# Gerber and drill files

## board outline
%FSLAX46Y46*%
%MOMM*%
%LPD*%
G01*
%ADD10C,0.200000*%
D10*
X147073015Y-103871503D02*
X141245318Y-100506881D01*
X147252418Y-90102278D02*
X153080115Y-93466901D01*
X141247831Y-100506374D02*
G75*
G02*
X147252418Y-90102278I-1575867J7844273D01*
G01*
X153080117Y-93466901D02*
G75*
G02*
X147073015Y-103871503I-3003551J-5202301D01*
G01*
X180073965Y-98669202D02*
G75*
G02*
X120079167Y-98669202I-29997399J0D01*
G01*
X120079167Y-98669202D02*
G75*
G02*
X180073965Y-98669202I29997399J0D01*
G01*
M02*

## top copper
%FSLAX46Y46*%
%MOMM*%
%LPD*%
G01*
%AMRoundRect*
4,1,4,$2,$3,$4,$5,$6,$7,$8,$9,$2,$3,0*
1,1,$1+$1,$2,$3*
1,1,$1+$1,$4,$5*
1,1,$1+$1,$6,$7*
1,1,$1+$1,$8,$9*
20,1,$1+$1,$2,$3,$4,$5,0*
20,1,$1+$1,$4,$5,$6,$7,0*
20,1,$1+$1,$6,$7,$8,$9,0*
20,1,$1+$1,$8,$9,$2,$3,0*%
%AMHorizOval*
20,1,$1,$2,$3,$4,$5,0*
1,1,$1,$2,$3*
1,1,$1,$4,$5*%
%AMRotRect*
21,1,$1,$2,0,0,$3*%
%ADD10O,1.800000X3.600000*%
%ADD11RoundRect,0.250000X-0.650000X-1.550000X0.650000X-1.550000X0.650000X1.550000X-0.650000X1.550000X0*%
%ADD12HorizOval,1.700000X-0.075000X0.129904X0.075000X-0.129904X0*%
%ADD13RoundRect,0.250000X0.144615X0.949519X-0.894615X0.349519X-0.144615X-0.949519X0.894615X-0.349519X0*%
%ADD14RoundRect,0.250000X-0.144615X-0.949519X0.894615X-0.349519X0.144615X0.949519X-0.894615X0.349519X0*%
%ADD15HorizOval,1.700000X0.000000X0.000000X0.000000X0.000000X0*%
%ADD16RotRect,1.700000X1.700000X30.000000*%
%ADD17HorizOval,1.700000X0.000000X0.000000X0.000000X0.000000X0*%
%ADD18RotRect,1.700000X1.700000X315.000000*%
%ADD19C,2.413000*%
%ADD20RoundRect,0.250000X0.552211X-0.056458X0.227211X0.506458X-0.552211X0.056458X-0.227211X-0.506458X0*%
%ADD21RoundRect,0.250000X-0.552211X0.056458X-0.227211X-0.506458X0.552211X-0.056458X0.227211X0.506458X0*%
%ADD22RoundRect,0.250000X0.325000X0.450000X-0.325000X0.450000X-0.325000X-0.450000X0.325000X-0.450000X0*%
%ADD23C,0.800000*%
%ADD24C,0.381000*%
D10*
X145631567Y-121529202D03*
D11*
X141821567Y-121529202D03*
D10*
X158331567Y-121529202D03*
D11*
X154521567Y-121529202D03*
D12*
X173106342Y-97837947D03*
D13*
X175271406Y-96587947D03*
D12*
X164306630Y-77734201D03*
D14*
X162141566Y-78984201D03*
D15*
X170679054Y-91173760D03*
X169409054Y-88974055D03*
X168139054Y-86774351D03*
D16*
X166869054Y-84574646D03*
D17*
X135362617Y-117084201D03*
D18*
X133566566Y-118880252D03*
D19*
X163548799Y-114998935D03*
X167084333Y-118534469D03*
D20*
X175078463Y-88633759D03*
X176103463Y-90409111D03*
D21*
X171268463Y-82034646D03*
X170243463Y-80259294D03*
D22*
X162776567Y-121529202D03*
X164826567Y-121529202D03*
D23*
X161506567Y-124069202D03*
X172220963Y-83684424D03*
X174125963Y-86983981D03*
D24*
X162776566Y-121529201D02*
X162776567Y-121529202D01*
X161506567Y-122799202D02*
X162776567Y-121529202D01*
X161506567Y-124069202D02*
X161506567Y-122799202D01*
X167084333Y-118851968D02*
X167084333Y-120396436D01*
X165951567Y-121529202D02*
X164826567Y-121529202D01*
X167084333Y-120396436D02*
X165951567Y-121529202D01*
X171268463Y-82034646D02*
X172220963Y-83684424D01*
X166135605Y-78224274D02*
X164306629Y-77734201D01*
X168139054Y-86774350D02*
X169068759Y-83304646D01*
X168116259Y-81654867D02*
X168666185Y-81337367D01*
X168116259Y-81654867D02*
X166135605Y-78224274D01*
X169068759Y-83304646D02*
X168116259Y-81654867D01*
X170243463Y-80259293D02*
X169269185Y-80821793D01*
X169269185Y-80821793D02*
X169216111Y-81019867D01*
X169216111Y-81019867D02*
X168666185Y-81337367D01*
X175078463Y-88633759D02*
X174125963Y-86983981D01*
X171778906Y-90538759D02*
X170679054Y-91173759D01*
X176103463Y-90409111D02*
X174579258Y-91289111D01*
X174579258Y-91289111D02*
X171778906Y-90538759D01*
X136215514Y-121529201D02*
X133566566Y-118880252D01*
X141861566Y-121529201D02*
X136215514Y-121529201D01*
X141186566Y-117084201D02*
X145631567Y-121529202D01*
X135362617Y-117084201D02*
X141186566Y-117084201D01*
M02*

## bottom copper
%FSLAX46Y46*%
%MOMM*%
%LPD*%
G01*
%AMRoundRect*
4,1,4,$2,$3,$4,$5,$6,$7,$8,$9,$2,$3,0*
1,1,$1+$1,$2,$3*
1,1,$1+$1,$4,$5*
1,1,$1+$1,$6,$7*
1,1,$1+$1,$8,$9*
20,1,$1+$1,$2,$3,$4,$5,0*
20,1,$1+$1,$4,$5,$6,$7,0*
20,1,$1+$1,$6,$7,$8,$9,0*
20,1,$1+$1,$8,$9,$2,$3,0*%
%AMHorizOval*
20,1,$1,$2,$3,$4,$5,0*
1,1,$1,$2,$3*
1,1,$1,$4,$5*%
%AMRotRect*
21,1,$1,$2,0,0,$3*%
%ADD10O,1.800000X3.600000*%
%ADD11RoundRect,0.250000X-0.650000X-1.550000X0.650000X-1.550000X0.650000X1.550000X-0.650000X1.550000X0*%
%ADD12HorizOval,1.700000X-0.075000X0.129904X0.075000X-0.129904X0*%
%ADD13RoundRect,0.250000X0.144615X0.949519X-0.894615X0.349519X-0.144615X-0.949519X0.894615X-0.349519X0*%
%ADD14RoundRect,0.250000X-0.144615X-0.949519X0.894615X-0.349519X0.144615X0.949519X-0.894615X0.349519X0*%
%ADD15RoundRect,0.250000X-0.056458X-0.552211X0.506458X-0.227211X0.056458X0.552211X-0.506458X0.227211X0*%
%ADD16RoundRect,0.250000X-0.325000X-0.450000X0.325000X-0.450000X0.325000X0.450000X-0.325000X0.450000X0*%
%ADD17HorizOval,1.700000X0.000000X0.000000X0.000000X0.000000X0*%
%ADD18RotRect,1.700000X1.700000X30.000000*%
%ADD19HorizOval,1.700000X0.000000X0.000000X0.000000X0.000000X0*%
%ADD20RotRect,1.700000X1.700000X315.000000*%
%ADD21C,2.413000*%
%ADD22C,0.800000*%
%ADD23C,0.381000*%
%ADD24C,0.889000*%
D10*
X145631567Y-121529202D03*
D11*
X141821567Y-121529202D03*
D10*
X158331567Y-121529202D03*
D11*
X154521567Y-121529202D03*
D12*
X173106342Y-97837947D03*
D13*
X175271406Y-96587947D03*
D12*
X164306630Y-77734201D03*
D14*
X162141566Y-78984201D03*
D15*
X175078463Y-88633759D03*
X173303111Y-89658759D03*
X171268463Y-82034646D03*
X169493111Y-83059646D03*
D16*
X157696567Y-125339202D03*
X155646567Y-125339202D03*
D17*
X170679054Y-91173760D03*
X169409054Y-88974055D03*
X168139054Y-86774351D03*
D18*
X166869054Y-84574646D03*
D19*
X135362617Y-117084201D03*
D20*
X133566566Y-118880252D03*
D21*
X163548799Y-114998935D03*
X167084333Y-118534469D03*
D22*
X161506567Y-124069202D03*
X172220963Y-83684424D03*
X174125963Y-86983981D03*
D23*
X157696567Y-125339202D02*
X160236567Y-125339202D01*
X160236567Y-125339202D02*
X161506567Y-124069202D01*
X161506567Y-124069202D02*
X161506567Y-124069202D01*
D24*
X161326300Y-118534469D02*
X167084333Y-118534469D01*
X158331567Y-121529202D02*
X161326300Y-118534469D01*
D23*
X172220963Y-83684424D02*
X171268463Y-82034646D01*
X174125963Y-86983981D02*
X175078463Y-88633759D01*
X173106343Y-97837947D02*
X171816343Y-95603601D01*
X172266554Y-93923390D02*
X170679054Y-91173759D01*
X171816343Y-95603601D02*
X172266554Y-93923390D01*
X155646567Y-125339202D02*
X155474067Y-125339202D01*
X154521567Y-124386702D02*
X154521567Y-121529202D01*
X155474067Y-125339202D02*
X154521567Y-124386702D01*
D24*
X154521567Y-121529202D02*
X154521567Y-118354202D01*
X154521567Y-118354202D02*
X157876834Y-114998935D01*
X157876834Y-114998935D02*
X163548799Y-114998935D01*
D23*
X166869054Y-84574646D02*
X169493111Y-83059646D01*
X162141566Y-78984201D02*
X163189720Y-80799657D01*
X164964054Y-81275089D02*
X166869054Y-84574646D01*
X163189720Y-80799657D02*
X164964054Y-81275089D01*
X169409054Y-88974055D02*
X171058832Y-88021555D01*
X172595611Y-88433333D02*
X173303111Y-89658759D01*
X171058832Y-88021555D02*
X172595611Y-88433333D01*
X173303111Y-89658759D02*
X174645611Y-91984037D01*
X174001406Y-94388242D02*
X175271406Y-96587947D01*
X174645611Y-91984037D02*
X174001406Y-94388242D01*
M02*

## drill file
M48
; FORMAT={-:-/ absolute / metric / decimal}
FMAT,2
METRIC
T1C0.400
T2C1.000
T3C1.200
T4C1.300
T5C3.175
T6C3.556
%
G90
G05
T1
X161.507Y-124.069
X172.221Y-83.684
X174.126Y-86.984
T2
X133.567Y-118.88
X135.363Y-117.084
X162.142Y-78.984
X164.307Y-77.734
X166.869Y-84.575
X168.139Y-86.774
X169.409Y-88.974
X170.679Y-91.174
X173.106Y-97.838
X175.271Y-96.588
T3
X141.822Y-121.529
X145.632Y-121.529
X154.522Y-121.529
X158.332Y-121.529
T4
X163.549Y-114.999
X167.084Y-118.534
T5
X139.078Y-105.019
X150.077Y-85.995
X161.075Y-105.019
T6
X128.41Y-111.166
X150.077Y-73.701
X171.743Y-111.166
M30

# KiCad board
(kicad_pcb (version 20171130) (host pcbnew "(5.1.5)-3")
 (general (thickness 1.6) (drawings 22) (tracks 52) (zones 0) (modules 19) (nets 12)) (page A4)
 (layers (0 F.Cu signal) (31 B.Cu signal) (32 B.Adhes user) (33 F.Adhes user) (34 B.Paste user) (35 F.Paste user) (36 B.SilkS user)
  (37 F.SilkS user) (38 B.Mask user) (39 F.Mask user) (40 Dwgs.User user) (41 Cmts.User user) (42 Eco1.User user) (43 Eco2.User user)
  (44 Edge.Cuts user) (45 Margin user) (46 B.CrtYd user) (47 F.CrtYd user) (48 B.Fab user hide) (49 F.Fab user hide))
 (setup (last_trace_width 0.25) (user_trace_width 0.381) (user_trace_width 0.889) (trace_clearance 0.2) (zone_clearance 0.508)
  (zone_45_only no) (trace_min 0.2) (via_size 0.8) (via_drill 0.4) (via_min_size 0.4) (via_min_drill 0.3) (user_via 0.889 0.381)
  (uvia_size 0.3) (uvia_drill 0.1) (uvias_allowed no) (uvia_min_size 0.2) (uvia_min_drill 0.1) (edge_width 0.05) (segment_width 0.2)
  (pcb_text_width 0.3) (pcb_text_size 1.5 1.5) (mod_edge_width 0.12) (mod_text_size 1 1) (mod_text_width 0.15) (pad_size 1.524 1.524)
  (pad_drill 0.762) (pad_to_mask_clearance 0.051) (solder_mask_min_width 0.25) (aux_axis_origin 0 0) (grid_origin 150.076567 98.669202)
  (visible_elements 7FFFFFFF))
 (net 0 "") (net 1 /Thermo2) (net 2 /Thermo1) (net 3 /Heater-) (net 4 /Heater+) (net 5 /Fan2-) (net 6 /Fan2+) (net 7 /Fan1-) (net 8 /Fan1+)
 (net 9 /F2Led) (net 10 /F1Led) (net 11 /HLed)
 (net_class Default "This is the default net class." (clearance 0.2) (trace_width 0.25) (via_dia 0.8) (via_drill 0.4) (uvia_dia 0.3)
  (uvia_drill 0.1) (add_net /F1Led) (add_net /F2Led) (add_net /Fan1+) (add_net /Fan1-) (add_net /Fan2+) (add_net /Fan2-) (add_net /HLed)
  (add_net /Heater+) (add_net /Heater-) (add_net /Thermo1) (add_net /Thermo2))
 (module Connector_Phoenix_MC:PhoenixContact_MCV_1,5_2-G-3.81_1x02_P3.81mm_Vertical (layer F.Cu) (at 141.821567 121.529202)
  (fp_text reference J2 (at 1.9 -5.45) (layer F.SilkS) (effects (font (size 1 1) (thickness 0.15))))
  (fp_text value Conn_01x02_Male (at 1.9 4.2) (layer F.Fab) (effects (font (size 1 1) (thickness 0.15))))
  (pad 2 thru_hole oval (at 3.81 0) (size 1.8 3.6) (drill 1.2) (layers *.Cu *.Mask) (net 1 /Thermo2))
  (pad 1 thru_hole roundrect (at 0 0) (size 1.8 3.6) (drill 1.2) (layers *.Cu *.Mask) (roundrect_rratio 0.138889) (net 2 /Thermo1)))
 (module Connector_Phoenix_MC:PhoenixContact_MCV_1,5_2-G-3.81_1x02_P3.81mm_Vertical (layer F.Cu) (at 154.521567 121.529202)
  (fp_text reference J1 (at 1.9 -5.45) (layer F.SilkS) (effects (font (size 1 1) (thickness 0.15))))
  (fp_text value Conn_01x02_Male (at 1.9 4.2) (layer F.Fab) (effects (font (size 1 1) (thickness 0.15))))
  (pad 2 thru_hole oval (at 3.81 0) (size 1.8 3.6) (drill 1.2) (layers *.Cu *.Mask) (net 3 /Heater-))
  (pad 1 thru_hole roundrect (at 0 0) (size 1.8 3.6) (drill 1.2) (layers *.Cu *.Mask) (roundrect_rratio 0.138889) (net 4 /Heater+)))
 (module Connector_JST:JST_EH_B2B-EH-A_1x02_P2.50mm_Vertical (layer F.Cu) (at 175.271406 96.587947 210)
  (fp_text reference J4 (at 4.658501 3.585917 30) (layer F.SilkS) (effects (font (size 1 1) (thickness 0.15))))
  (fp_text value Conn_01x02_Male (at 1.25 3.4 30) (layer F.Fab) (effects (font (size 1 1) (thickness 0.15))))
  (pad 2 thru_hole oval (at 2.5 0 210) (size 1.7 2) (drill 1) (layers *.Cu *.Mask) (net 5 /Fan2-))
  (pad 1 thru_hole roundrect (at 0 0 210) (size 1.7 2) (drill 1) (layers *.Cu *.Mask) (roundrect_rratio 0.147059) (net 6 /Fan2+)))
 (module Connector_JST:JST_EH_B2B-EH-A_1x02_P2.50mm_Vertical (layer F.Cu) (at 162.141566 78.984201 30)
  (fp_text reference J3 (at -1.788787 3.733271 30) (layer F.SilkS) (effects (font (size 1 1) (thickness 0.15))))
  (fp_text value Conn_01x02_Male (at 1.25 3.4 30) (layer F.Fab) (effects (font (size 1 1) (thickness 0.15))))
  (pad 2 thru_hole oval (at 2.5 0 30) (size 1.7 2) (drill 1) (layers *.Cu *.Mask) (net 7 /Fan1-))
  (pad 1 thru_hole roundrect (at 0 0 30) (size 1.7 2) (drill 1) (layers *.Cu *.Mask) (roundrect_rratio 0.147059) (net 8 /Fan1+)))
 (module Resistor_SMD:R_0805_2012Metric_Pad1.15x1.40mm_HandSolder (layer B.Cu) (at 174.190787 89.146259 30)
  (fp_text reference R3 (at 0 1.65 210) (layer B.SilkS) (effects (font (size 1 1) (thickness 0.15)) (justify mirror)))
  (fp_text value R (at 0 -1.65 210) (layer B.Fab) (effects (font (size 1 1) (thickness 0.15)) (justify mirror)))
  (pad 2 smd roundrect (at 1.025 0 30) (size 1.15 1.4) (layers B.Cu B.Paste B.Mask) (roundrect_rratio 0.217391) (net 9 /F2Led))
  (pad 1 smd roundrect (at -1.025 0 30) (size 1.15 1.4) (layers B.Cu B.Paste B.Mask) (roundrect_rratio 0.217391) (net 6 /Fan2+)))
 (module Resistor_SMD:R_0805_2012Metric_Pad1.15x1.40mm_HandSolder (layer B.Cu) (at 170.380787 82.547146 30)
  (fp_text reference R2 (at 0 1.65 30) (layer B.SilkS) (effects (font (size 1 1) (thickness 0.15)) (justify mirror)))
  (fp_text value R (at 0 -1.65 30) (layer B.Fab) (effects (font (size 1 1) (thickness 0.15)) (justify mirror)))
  (pad 2 smd roundrect (at 1.025 0 30) (size 1.15 1.4) (layers B.Cu B.Paste B.Mask) (roundrect_rratio 0.217391) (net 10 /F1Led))
  (pad 1 smd roundrect (at -1.025 0 30) (size 1.15 1.4) (layers B.Cu B.Paste B.Mask) (roundrect_rratio 0.217391) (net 8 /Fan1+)))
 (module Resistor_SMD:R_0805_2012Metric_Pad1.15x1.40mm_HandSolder (layer B.Cu) (at 156.671567 125.339202)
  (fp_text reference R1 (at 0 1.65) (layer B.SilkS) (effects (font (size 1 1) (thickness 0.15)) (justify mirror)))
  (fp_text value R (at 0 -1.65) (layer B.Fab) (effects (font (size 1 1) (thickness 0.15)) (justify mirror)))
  (pad 2 smd roundrect (at 1.025 0) (size 1.15 1.4) (layers B.Cu B.Paste B.Mask) (roundrect_rratio 0.217391) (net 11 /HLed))
  (pad 1 smd roundrect (at -1.025 0) (size 1.15 1.4) (layers B.Cu B.Paste B.Mask) (roundrect_rratio 0.217391) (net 4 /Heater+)))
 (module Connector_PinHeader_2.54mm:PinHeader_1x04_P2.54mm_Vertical (layer F.Cu) (at 166.869054 84.574646 30)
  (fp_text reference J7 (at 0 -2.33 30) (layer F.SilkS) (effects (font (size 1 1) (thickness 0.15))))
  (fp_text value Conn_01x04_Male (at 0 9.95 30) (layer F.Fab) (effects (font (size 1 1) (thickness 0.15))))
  (pad 4 thru_hole oval (at 0 7.62 30) (size 1.7 1.7) (drill 1) (layers *.Cu *.Mask) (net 5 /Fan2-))
  (pad 3 thru_hole oval (at 0 5.08 30) (size 1.7 1.7) (drill 1) (layers *.Cu *.Mask) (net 6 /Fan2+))
  (pad 2 thru_hole oval (at 0 2.54 30) (size 1.7 1.7) (drill 1) (layers *.Cu *.Mask) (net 7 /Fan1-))
  (pad 1 thru_hole rect (at 0 0 30) (size 1.7 1.7) (drill 1) (layers *.Cu *.Mask) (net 8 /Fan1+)))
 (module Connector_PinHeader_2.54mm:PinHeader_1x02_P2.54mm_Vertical (layer B.Cu) (at 133.566566 118.880252 315)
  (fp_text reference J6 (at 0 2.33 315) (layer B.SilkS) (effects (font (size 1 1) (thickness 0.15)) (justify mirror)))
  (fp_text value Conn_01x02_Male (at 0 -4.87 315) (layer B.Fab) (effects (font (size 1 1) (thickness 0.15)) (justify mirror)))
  (pad 2 thru_hole oval (at 0 -2.54 315) (size 1.7 1.7) (drill 1) (layers *.Cu *.Mask) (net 1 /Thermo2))
  (pad 1 thru_hole rect (at 0 0 315) (size 1.7 1.7) (drill 1) (layers *.Cu *.Mask) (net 2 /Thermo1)))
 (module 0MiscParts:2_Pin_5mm (layer B.Cu) (at 165.316566 116.766702 315)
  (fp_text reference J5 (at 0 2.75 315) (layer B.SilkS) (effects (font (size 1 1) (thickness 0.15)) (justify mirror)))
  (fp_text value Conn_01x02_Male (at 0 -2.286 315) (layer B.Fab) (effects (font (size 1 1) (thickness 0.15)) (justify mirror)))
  (pad 1 thru_hole circle (at -2.5 0 315) (size 2.413 2.413) (drill 1.3) (layers *.Cu *.Mask) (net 4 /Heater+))
  (pad 2 thru_hole circle (at 2.5 0 315) (size 2.413 2.413) (drill 1.3) (layers *.Cu *.Mask) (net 3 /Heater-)))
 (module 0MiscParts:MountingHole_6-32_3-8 (layer F.Cu) (at 128.410365 111.166002)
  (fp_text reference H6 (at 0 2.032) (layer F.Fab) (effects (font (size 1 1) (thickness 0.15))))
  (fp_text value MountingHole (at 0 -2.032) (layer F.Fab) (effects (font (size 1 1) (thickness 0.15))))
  (pad "" np_thru_hole circle (at 0 0) (size 3.556 3.556) (drill 3.556) (layers *.Cu *.Mask)))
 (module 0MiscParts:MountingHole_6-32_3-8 (layer F.Cu) (at 150.076566 73.701003)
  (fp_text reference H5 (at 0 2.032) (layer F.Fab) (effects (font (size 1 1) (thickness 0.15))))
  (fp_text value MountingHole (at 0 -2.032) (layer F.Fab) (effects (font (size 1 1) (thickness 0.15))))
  (pad "" np_thru_hole circle (at 0 0) (size 3.556 3.556) (drill 3.556) (layers *.Cu *.Mask)))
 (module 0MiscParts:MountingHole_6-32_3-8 (layer F.Cu) (at 171.742766 111.166003)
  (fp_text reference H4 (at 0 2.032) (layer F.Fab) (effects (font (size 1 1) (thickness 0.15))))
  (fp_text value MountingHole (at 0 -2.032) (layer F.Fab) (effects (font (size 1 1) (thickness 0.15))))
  (pad "" np_thru_hole circle (at 0 0) (size 3.556 3.556) (drill 3.556) (layers *.Cu *.Mask)))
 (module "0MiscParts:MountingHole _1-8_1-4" (layer F.Cu) (at 139.078365 105.019202)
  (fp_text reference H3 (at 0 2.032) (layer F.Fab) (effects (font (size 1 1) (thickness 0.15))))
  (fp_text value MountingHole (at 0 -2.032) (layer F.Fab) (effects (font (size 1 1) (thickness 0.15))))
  (pad "" np_thru_hole circle (at 0 0) (size 3.175 3.175) (drill 3.175) (layers *.Cu *.Mask)))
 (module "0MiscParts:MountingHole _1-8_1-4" (layer F.Cu) (at 161.074767 105.019201)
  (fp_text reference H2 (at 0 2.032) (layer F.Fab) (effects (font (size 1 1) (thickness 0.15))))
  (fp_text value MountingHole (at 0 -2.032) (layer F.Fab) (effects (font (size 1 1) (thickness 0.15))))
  (pad "" np_thru_hole circle (at 0 0) (size 3.175 3.175) (drill 3.175) (layers *.Cu *.Mask)))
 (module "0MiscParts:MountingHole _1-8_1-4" (layer F.Cu) (at 150.076565 85.994602)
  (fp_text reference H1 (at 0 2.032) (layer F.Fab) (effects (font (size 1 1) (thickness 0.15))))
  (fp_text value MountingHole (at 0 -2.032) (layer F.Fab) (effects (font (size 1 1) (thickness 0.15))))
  (pad "" np_thru_hole circle (at 0 0) (size 3.175 3.175) (drill 3.175) (layers *.Cu *.Mask)))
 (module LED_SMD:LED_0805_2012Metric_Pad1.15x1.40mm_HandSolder (layer F.Cu) (at 175.590963 89.521435 120)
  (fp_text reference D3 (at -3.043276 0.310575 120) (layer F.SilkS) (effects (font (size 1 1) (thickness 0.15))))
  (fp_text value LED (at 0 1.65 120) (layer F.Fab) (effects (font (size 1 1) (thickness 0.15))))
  (pad 2 smd roundrect (at 1.025 0 120) (size 1.15 1.4) (layers F.Cu F.Paste F.Mask) (roundrect_rratio 0.217391) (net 9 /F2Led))
  (pad 1 smd roundrect (at -1.025 0 120) (size 1.15 1.4) (layers F.Cu F.Paste F.Mask) (roundrect_rratio 0.217391) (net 5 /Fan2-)))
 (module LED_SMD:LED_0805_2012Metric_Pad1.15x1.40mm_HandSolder (layer F.Cu) (at 170.755963 81.14697 300)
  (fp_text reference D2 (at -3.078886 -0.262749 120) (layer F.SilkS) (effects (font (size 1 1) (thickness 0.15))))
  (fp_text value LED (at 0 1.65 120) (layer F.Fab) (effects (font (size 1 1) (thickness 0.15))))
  (pad 2 smd roundrect (at 1.025 0 300) (size 1.15 1.4) (layers F.Cu F.Paste F.Mask) (roundrect_rratio 0.217391) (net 10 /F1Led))
  (pad 1 smd roundrect (at -1.025 0 300) (size 1.15 1.4) (layers F.Cu F.Paste F.Mask) (roundrect_rratio 0.217391) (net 7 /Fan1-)))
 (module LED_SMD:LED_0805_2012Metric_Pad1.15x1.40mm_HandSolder (layer F.Cu) (at 163.801567 121.529202 180)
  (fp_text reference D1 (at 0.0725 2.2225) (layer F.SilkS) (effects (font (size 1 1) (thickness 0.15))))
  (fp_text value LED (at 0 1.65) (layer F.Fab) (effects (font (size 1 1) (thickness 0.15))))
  (pad 2 smd roundrect (at 1.025 0 180) (size 1.15 1.4) (layers F.Cu F.Paste F.Mask) (roundrect_rratio 0.217391) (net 11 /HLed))
  (pad 1 smd roundrect (at -1.025 0 180) (size 1.15 1.4) (layers F.Cu F.Paste F.Mask) (roundrect_rratio 0.217391) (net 3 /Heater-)))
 (gr_line (start 147.073015 103.871503) (end 141.245318 100.506881) (layer Edge.Cuts) (width 0.2))
 (gr_line (start 147.252418 90.102278) (end 153.080115 93.466901) (layer Edge.Cuts) (width 0.2))
 (gr_arc (start 139.671964 92.662101) (end 147.252418 90.102278) (angle -262.7) (layer Edge.Cuts) (width 0.2))
 (gr_arc (start 150.076566 98.669202) (end 147.073015 103.871503) (angle -180) (layer Edge.Cuts) (width 0.2))
 (gr_circle (center 150.076566 98.669202) (end 180.073965 98.669203) (layer Edge.Cuts) (width 0.2))
 (segment (start 162.776566 121.529201) (end 162.776567 121.529202) (width 0.381) (layer F.Cu) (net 11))
 (segment (start 157.696567 125.339202) (end 160.236567 125.339202) (width 0.381) (layer B.Cu) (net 11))
 (segment (start 160.236567 125.339202) (end 161.506567 124.069202) (width 0.381) (layer B.Cu) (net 11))
 (segment (start 161.506567 124.069202) (end 161.506567 124.069202) (width 0.381) (layer B.Cu) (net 11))
 (via (at 161.506567 124.069202) (size 0.8) (drill 0.4) (layers F.Cu B.Cu) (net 11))
 (segment (start 161.506567 122.799202) (end 162.776567 121.529202) (width 0.381) (layer F.Cu) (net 11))
 (segment (start 161.506567 124.069202) (end 161.506567 122.799202) (width 0.381) (layer F.Cu) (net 11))
 (segment (start 167.084333 118.851968) (end 167.084333 120.396436) (width 0.381) (layer F.Cu) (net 3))
 (segment (start 165.951567 121.529202) (end 164.826567 121.529202) (width 0.381) (layer F.Cu) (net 3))
 (segment (start 167.084333 120.396436) (end 165.951567 121.529202) (width 0.381) (layer F.Cu) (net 3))
 (segment (start 161.3263 118.534469) (end 167.084333 118.534469) (width 0.889) (layer B.Cu) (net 3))
 (segment (start 158.331567 121.529202) (end 161.3263 118.534469) (width 0.889) (layer B.Cu) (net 3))
 (via (at 172.220963 83.684424) (size 0.8) (drill 0.4) (layers F.Cu B.Cu) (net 10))
 (segment (start 171.268463 82.034646) (end 172.220963 83.684424) (width 0.381) (layer F.Cu) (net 10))
 (segment (start 172.220963 83.684424) (end 171.268463 82.034646) (width 0.381) (layer B.Cu) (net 10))
 (segment (start 166.135605 78.224274) (end 164.306629 77.734201) (width 0.381) (layer F.Cu) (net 7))
 (segment (start 168.139054 86.77435) (end 169.068759 83.304646) (width 0.381) (layer F.Cu) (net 7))
 (segment (start 168.116259 81.654867) (end 168.666185 81.337367) (width 0.381) (layer F.Cu) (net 7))
 (segment (start 168.116259 81.654867) (end 166.135605 78.224274) (width 0.381) (layer F.Cu) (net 7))
 (segment (start 169.068759 83.304646) (end 168.116259 81.654867) (width 0.381) (layer F.Cu) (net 7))
 (segment (start 170.243463 80.259293) (end 169.269185 80.821793) (width 0.381) (layer F.Cu) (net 7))
 (segment (start 169.269185 80.821793) (end 169.216111 81.019867) (width 0.381) (layer F.Cu) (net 7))
 (segment (start 169.216111 81.019867) (end 168.666185 81.337367) (width 0.381) (layer F.Cu) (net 7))
 (via (at 174.125963 86.983981) (size 0.8) (drill 0.4) (layers F.Cu B.Cu) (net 9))
 (segment (start 175.078463 88.633759) (end 174.125963 86.983981) (width 0.381) (layer F.Cu) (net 9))
 (segment (start 174.125963 86.983981) (end 175.078463 88.633759) (width 0.381) (layer B.Cu) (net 9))
 (segment (start 173.106343 97.837947) (end 171.816343 95.603601) (width 0.381) (layer B.Cu) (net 5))
 (segment (start 172.266554 93.92339) (end 170.679054 91.173759) (width 0.381) (layer B.Cu) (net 5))
 (segment (start 171.816343 95.603601) (end 172.266554 93.92339) (width 0.381) (layer B.Cu) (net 5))
 (segment (start 171.778906 90.538759) (end 170.679054 91.173759) (width 0.381) (layer F.Cu) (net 5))
 (segment (start 176.103463 90.409111) (end 174.579258 91.289111) (width 0.381) (layer F.Cu) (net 5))
 (segment (start 174.579258 91.289111) (end 171.778906 90.538759) (width 0.381) (layer F.Cu) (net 5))
 (segment (start 155.646567 125.339202) (end 155.474067 125.339202) (width 0.381) (layer B.Cu) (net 4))
 (segment (start 154.521567 124.386702) (end 154.521567 121.529202) (width 0.381) (layer B.Cu) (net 4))
 (segment (start 155.474067 125.339202) (end 154.521567 124.386702) (width 0.381) (layer B.Cu) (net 4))
 (segment (start 154.521567 121.529202) (end 154.521567 118.354202) (width 0.889) (layer B.Cu) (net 4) (status 1000000))
 (segment (start 154.521567 118.354202) (end 157.876834 114.998935) (width 0.889) (layer B.Cu) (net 4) (status 1000000))
 (segment (start 157.876834 114.998935) (end 163.548799 114.998935) (width 0.889) (layer B.Cu) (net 4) (status 1000000))
 (segment (start 136.215514 121.529201) (end 133.566566 118.880252) (width 0.381) (layer F.Cu) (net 2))
 (segment (start 141.861566 121.529201) (end 136.215514 121.529201) (width 0.381) (layer F.Cu) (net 2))
 (segment (start 141.186566 117.084201) (end 145.631567 121.529202) (width 0.381) (layer F.Cu) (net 1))
 (segment (start 135.362617 117.084201) (end 141.186566 117.084201) (width 0.381) (layer F.Cu) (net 1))
 (segment (start 166.869054 84.574646) (end 169.493111 83.059646) (width 0.381) (layer B.Cu) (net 8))
 (segment (start 162.141566 78.984201) (end 163.18972 80.799657) (width 0.381) (layer B.Cu) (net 8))
 (segment (start 164.964054 81.275089) (end 166.869054 84.574646) (width 0.381) (layer B.Cu) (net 8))
 (segment (start 163.18972 80.799657) (end 164.964054 81.275089) (width 0.381) (layer B.Cu) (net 8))
 (segment (start 169.409054 88.974055) (end 171.058832 88.021555) (width 0.381) (layer B.Cu) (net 6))
 (segment (start 172.595611 88.433333) (end 173.303111 89.658759) (width 0.381) (layer B.Cu) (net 6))
 (segment (start 171.058832 88.021555) (end 172.595611 88.433333) (width 0.381) (layer B.Cu) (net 6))
 (segment (start 173.303111 89.658759) (end 174.645611 91.984037) (width 0.381) (layer B.Cu) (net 6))
 (segment (start 174.001406 94.388242) (end 175.271406 96.587947) (width 0.381) (layer B.Cu) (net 6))
 (segment (start 174.645611 91.984037) (end 174.001406 94.388242) (width 0.381) (layer B.Cu) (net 6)))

